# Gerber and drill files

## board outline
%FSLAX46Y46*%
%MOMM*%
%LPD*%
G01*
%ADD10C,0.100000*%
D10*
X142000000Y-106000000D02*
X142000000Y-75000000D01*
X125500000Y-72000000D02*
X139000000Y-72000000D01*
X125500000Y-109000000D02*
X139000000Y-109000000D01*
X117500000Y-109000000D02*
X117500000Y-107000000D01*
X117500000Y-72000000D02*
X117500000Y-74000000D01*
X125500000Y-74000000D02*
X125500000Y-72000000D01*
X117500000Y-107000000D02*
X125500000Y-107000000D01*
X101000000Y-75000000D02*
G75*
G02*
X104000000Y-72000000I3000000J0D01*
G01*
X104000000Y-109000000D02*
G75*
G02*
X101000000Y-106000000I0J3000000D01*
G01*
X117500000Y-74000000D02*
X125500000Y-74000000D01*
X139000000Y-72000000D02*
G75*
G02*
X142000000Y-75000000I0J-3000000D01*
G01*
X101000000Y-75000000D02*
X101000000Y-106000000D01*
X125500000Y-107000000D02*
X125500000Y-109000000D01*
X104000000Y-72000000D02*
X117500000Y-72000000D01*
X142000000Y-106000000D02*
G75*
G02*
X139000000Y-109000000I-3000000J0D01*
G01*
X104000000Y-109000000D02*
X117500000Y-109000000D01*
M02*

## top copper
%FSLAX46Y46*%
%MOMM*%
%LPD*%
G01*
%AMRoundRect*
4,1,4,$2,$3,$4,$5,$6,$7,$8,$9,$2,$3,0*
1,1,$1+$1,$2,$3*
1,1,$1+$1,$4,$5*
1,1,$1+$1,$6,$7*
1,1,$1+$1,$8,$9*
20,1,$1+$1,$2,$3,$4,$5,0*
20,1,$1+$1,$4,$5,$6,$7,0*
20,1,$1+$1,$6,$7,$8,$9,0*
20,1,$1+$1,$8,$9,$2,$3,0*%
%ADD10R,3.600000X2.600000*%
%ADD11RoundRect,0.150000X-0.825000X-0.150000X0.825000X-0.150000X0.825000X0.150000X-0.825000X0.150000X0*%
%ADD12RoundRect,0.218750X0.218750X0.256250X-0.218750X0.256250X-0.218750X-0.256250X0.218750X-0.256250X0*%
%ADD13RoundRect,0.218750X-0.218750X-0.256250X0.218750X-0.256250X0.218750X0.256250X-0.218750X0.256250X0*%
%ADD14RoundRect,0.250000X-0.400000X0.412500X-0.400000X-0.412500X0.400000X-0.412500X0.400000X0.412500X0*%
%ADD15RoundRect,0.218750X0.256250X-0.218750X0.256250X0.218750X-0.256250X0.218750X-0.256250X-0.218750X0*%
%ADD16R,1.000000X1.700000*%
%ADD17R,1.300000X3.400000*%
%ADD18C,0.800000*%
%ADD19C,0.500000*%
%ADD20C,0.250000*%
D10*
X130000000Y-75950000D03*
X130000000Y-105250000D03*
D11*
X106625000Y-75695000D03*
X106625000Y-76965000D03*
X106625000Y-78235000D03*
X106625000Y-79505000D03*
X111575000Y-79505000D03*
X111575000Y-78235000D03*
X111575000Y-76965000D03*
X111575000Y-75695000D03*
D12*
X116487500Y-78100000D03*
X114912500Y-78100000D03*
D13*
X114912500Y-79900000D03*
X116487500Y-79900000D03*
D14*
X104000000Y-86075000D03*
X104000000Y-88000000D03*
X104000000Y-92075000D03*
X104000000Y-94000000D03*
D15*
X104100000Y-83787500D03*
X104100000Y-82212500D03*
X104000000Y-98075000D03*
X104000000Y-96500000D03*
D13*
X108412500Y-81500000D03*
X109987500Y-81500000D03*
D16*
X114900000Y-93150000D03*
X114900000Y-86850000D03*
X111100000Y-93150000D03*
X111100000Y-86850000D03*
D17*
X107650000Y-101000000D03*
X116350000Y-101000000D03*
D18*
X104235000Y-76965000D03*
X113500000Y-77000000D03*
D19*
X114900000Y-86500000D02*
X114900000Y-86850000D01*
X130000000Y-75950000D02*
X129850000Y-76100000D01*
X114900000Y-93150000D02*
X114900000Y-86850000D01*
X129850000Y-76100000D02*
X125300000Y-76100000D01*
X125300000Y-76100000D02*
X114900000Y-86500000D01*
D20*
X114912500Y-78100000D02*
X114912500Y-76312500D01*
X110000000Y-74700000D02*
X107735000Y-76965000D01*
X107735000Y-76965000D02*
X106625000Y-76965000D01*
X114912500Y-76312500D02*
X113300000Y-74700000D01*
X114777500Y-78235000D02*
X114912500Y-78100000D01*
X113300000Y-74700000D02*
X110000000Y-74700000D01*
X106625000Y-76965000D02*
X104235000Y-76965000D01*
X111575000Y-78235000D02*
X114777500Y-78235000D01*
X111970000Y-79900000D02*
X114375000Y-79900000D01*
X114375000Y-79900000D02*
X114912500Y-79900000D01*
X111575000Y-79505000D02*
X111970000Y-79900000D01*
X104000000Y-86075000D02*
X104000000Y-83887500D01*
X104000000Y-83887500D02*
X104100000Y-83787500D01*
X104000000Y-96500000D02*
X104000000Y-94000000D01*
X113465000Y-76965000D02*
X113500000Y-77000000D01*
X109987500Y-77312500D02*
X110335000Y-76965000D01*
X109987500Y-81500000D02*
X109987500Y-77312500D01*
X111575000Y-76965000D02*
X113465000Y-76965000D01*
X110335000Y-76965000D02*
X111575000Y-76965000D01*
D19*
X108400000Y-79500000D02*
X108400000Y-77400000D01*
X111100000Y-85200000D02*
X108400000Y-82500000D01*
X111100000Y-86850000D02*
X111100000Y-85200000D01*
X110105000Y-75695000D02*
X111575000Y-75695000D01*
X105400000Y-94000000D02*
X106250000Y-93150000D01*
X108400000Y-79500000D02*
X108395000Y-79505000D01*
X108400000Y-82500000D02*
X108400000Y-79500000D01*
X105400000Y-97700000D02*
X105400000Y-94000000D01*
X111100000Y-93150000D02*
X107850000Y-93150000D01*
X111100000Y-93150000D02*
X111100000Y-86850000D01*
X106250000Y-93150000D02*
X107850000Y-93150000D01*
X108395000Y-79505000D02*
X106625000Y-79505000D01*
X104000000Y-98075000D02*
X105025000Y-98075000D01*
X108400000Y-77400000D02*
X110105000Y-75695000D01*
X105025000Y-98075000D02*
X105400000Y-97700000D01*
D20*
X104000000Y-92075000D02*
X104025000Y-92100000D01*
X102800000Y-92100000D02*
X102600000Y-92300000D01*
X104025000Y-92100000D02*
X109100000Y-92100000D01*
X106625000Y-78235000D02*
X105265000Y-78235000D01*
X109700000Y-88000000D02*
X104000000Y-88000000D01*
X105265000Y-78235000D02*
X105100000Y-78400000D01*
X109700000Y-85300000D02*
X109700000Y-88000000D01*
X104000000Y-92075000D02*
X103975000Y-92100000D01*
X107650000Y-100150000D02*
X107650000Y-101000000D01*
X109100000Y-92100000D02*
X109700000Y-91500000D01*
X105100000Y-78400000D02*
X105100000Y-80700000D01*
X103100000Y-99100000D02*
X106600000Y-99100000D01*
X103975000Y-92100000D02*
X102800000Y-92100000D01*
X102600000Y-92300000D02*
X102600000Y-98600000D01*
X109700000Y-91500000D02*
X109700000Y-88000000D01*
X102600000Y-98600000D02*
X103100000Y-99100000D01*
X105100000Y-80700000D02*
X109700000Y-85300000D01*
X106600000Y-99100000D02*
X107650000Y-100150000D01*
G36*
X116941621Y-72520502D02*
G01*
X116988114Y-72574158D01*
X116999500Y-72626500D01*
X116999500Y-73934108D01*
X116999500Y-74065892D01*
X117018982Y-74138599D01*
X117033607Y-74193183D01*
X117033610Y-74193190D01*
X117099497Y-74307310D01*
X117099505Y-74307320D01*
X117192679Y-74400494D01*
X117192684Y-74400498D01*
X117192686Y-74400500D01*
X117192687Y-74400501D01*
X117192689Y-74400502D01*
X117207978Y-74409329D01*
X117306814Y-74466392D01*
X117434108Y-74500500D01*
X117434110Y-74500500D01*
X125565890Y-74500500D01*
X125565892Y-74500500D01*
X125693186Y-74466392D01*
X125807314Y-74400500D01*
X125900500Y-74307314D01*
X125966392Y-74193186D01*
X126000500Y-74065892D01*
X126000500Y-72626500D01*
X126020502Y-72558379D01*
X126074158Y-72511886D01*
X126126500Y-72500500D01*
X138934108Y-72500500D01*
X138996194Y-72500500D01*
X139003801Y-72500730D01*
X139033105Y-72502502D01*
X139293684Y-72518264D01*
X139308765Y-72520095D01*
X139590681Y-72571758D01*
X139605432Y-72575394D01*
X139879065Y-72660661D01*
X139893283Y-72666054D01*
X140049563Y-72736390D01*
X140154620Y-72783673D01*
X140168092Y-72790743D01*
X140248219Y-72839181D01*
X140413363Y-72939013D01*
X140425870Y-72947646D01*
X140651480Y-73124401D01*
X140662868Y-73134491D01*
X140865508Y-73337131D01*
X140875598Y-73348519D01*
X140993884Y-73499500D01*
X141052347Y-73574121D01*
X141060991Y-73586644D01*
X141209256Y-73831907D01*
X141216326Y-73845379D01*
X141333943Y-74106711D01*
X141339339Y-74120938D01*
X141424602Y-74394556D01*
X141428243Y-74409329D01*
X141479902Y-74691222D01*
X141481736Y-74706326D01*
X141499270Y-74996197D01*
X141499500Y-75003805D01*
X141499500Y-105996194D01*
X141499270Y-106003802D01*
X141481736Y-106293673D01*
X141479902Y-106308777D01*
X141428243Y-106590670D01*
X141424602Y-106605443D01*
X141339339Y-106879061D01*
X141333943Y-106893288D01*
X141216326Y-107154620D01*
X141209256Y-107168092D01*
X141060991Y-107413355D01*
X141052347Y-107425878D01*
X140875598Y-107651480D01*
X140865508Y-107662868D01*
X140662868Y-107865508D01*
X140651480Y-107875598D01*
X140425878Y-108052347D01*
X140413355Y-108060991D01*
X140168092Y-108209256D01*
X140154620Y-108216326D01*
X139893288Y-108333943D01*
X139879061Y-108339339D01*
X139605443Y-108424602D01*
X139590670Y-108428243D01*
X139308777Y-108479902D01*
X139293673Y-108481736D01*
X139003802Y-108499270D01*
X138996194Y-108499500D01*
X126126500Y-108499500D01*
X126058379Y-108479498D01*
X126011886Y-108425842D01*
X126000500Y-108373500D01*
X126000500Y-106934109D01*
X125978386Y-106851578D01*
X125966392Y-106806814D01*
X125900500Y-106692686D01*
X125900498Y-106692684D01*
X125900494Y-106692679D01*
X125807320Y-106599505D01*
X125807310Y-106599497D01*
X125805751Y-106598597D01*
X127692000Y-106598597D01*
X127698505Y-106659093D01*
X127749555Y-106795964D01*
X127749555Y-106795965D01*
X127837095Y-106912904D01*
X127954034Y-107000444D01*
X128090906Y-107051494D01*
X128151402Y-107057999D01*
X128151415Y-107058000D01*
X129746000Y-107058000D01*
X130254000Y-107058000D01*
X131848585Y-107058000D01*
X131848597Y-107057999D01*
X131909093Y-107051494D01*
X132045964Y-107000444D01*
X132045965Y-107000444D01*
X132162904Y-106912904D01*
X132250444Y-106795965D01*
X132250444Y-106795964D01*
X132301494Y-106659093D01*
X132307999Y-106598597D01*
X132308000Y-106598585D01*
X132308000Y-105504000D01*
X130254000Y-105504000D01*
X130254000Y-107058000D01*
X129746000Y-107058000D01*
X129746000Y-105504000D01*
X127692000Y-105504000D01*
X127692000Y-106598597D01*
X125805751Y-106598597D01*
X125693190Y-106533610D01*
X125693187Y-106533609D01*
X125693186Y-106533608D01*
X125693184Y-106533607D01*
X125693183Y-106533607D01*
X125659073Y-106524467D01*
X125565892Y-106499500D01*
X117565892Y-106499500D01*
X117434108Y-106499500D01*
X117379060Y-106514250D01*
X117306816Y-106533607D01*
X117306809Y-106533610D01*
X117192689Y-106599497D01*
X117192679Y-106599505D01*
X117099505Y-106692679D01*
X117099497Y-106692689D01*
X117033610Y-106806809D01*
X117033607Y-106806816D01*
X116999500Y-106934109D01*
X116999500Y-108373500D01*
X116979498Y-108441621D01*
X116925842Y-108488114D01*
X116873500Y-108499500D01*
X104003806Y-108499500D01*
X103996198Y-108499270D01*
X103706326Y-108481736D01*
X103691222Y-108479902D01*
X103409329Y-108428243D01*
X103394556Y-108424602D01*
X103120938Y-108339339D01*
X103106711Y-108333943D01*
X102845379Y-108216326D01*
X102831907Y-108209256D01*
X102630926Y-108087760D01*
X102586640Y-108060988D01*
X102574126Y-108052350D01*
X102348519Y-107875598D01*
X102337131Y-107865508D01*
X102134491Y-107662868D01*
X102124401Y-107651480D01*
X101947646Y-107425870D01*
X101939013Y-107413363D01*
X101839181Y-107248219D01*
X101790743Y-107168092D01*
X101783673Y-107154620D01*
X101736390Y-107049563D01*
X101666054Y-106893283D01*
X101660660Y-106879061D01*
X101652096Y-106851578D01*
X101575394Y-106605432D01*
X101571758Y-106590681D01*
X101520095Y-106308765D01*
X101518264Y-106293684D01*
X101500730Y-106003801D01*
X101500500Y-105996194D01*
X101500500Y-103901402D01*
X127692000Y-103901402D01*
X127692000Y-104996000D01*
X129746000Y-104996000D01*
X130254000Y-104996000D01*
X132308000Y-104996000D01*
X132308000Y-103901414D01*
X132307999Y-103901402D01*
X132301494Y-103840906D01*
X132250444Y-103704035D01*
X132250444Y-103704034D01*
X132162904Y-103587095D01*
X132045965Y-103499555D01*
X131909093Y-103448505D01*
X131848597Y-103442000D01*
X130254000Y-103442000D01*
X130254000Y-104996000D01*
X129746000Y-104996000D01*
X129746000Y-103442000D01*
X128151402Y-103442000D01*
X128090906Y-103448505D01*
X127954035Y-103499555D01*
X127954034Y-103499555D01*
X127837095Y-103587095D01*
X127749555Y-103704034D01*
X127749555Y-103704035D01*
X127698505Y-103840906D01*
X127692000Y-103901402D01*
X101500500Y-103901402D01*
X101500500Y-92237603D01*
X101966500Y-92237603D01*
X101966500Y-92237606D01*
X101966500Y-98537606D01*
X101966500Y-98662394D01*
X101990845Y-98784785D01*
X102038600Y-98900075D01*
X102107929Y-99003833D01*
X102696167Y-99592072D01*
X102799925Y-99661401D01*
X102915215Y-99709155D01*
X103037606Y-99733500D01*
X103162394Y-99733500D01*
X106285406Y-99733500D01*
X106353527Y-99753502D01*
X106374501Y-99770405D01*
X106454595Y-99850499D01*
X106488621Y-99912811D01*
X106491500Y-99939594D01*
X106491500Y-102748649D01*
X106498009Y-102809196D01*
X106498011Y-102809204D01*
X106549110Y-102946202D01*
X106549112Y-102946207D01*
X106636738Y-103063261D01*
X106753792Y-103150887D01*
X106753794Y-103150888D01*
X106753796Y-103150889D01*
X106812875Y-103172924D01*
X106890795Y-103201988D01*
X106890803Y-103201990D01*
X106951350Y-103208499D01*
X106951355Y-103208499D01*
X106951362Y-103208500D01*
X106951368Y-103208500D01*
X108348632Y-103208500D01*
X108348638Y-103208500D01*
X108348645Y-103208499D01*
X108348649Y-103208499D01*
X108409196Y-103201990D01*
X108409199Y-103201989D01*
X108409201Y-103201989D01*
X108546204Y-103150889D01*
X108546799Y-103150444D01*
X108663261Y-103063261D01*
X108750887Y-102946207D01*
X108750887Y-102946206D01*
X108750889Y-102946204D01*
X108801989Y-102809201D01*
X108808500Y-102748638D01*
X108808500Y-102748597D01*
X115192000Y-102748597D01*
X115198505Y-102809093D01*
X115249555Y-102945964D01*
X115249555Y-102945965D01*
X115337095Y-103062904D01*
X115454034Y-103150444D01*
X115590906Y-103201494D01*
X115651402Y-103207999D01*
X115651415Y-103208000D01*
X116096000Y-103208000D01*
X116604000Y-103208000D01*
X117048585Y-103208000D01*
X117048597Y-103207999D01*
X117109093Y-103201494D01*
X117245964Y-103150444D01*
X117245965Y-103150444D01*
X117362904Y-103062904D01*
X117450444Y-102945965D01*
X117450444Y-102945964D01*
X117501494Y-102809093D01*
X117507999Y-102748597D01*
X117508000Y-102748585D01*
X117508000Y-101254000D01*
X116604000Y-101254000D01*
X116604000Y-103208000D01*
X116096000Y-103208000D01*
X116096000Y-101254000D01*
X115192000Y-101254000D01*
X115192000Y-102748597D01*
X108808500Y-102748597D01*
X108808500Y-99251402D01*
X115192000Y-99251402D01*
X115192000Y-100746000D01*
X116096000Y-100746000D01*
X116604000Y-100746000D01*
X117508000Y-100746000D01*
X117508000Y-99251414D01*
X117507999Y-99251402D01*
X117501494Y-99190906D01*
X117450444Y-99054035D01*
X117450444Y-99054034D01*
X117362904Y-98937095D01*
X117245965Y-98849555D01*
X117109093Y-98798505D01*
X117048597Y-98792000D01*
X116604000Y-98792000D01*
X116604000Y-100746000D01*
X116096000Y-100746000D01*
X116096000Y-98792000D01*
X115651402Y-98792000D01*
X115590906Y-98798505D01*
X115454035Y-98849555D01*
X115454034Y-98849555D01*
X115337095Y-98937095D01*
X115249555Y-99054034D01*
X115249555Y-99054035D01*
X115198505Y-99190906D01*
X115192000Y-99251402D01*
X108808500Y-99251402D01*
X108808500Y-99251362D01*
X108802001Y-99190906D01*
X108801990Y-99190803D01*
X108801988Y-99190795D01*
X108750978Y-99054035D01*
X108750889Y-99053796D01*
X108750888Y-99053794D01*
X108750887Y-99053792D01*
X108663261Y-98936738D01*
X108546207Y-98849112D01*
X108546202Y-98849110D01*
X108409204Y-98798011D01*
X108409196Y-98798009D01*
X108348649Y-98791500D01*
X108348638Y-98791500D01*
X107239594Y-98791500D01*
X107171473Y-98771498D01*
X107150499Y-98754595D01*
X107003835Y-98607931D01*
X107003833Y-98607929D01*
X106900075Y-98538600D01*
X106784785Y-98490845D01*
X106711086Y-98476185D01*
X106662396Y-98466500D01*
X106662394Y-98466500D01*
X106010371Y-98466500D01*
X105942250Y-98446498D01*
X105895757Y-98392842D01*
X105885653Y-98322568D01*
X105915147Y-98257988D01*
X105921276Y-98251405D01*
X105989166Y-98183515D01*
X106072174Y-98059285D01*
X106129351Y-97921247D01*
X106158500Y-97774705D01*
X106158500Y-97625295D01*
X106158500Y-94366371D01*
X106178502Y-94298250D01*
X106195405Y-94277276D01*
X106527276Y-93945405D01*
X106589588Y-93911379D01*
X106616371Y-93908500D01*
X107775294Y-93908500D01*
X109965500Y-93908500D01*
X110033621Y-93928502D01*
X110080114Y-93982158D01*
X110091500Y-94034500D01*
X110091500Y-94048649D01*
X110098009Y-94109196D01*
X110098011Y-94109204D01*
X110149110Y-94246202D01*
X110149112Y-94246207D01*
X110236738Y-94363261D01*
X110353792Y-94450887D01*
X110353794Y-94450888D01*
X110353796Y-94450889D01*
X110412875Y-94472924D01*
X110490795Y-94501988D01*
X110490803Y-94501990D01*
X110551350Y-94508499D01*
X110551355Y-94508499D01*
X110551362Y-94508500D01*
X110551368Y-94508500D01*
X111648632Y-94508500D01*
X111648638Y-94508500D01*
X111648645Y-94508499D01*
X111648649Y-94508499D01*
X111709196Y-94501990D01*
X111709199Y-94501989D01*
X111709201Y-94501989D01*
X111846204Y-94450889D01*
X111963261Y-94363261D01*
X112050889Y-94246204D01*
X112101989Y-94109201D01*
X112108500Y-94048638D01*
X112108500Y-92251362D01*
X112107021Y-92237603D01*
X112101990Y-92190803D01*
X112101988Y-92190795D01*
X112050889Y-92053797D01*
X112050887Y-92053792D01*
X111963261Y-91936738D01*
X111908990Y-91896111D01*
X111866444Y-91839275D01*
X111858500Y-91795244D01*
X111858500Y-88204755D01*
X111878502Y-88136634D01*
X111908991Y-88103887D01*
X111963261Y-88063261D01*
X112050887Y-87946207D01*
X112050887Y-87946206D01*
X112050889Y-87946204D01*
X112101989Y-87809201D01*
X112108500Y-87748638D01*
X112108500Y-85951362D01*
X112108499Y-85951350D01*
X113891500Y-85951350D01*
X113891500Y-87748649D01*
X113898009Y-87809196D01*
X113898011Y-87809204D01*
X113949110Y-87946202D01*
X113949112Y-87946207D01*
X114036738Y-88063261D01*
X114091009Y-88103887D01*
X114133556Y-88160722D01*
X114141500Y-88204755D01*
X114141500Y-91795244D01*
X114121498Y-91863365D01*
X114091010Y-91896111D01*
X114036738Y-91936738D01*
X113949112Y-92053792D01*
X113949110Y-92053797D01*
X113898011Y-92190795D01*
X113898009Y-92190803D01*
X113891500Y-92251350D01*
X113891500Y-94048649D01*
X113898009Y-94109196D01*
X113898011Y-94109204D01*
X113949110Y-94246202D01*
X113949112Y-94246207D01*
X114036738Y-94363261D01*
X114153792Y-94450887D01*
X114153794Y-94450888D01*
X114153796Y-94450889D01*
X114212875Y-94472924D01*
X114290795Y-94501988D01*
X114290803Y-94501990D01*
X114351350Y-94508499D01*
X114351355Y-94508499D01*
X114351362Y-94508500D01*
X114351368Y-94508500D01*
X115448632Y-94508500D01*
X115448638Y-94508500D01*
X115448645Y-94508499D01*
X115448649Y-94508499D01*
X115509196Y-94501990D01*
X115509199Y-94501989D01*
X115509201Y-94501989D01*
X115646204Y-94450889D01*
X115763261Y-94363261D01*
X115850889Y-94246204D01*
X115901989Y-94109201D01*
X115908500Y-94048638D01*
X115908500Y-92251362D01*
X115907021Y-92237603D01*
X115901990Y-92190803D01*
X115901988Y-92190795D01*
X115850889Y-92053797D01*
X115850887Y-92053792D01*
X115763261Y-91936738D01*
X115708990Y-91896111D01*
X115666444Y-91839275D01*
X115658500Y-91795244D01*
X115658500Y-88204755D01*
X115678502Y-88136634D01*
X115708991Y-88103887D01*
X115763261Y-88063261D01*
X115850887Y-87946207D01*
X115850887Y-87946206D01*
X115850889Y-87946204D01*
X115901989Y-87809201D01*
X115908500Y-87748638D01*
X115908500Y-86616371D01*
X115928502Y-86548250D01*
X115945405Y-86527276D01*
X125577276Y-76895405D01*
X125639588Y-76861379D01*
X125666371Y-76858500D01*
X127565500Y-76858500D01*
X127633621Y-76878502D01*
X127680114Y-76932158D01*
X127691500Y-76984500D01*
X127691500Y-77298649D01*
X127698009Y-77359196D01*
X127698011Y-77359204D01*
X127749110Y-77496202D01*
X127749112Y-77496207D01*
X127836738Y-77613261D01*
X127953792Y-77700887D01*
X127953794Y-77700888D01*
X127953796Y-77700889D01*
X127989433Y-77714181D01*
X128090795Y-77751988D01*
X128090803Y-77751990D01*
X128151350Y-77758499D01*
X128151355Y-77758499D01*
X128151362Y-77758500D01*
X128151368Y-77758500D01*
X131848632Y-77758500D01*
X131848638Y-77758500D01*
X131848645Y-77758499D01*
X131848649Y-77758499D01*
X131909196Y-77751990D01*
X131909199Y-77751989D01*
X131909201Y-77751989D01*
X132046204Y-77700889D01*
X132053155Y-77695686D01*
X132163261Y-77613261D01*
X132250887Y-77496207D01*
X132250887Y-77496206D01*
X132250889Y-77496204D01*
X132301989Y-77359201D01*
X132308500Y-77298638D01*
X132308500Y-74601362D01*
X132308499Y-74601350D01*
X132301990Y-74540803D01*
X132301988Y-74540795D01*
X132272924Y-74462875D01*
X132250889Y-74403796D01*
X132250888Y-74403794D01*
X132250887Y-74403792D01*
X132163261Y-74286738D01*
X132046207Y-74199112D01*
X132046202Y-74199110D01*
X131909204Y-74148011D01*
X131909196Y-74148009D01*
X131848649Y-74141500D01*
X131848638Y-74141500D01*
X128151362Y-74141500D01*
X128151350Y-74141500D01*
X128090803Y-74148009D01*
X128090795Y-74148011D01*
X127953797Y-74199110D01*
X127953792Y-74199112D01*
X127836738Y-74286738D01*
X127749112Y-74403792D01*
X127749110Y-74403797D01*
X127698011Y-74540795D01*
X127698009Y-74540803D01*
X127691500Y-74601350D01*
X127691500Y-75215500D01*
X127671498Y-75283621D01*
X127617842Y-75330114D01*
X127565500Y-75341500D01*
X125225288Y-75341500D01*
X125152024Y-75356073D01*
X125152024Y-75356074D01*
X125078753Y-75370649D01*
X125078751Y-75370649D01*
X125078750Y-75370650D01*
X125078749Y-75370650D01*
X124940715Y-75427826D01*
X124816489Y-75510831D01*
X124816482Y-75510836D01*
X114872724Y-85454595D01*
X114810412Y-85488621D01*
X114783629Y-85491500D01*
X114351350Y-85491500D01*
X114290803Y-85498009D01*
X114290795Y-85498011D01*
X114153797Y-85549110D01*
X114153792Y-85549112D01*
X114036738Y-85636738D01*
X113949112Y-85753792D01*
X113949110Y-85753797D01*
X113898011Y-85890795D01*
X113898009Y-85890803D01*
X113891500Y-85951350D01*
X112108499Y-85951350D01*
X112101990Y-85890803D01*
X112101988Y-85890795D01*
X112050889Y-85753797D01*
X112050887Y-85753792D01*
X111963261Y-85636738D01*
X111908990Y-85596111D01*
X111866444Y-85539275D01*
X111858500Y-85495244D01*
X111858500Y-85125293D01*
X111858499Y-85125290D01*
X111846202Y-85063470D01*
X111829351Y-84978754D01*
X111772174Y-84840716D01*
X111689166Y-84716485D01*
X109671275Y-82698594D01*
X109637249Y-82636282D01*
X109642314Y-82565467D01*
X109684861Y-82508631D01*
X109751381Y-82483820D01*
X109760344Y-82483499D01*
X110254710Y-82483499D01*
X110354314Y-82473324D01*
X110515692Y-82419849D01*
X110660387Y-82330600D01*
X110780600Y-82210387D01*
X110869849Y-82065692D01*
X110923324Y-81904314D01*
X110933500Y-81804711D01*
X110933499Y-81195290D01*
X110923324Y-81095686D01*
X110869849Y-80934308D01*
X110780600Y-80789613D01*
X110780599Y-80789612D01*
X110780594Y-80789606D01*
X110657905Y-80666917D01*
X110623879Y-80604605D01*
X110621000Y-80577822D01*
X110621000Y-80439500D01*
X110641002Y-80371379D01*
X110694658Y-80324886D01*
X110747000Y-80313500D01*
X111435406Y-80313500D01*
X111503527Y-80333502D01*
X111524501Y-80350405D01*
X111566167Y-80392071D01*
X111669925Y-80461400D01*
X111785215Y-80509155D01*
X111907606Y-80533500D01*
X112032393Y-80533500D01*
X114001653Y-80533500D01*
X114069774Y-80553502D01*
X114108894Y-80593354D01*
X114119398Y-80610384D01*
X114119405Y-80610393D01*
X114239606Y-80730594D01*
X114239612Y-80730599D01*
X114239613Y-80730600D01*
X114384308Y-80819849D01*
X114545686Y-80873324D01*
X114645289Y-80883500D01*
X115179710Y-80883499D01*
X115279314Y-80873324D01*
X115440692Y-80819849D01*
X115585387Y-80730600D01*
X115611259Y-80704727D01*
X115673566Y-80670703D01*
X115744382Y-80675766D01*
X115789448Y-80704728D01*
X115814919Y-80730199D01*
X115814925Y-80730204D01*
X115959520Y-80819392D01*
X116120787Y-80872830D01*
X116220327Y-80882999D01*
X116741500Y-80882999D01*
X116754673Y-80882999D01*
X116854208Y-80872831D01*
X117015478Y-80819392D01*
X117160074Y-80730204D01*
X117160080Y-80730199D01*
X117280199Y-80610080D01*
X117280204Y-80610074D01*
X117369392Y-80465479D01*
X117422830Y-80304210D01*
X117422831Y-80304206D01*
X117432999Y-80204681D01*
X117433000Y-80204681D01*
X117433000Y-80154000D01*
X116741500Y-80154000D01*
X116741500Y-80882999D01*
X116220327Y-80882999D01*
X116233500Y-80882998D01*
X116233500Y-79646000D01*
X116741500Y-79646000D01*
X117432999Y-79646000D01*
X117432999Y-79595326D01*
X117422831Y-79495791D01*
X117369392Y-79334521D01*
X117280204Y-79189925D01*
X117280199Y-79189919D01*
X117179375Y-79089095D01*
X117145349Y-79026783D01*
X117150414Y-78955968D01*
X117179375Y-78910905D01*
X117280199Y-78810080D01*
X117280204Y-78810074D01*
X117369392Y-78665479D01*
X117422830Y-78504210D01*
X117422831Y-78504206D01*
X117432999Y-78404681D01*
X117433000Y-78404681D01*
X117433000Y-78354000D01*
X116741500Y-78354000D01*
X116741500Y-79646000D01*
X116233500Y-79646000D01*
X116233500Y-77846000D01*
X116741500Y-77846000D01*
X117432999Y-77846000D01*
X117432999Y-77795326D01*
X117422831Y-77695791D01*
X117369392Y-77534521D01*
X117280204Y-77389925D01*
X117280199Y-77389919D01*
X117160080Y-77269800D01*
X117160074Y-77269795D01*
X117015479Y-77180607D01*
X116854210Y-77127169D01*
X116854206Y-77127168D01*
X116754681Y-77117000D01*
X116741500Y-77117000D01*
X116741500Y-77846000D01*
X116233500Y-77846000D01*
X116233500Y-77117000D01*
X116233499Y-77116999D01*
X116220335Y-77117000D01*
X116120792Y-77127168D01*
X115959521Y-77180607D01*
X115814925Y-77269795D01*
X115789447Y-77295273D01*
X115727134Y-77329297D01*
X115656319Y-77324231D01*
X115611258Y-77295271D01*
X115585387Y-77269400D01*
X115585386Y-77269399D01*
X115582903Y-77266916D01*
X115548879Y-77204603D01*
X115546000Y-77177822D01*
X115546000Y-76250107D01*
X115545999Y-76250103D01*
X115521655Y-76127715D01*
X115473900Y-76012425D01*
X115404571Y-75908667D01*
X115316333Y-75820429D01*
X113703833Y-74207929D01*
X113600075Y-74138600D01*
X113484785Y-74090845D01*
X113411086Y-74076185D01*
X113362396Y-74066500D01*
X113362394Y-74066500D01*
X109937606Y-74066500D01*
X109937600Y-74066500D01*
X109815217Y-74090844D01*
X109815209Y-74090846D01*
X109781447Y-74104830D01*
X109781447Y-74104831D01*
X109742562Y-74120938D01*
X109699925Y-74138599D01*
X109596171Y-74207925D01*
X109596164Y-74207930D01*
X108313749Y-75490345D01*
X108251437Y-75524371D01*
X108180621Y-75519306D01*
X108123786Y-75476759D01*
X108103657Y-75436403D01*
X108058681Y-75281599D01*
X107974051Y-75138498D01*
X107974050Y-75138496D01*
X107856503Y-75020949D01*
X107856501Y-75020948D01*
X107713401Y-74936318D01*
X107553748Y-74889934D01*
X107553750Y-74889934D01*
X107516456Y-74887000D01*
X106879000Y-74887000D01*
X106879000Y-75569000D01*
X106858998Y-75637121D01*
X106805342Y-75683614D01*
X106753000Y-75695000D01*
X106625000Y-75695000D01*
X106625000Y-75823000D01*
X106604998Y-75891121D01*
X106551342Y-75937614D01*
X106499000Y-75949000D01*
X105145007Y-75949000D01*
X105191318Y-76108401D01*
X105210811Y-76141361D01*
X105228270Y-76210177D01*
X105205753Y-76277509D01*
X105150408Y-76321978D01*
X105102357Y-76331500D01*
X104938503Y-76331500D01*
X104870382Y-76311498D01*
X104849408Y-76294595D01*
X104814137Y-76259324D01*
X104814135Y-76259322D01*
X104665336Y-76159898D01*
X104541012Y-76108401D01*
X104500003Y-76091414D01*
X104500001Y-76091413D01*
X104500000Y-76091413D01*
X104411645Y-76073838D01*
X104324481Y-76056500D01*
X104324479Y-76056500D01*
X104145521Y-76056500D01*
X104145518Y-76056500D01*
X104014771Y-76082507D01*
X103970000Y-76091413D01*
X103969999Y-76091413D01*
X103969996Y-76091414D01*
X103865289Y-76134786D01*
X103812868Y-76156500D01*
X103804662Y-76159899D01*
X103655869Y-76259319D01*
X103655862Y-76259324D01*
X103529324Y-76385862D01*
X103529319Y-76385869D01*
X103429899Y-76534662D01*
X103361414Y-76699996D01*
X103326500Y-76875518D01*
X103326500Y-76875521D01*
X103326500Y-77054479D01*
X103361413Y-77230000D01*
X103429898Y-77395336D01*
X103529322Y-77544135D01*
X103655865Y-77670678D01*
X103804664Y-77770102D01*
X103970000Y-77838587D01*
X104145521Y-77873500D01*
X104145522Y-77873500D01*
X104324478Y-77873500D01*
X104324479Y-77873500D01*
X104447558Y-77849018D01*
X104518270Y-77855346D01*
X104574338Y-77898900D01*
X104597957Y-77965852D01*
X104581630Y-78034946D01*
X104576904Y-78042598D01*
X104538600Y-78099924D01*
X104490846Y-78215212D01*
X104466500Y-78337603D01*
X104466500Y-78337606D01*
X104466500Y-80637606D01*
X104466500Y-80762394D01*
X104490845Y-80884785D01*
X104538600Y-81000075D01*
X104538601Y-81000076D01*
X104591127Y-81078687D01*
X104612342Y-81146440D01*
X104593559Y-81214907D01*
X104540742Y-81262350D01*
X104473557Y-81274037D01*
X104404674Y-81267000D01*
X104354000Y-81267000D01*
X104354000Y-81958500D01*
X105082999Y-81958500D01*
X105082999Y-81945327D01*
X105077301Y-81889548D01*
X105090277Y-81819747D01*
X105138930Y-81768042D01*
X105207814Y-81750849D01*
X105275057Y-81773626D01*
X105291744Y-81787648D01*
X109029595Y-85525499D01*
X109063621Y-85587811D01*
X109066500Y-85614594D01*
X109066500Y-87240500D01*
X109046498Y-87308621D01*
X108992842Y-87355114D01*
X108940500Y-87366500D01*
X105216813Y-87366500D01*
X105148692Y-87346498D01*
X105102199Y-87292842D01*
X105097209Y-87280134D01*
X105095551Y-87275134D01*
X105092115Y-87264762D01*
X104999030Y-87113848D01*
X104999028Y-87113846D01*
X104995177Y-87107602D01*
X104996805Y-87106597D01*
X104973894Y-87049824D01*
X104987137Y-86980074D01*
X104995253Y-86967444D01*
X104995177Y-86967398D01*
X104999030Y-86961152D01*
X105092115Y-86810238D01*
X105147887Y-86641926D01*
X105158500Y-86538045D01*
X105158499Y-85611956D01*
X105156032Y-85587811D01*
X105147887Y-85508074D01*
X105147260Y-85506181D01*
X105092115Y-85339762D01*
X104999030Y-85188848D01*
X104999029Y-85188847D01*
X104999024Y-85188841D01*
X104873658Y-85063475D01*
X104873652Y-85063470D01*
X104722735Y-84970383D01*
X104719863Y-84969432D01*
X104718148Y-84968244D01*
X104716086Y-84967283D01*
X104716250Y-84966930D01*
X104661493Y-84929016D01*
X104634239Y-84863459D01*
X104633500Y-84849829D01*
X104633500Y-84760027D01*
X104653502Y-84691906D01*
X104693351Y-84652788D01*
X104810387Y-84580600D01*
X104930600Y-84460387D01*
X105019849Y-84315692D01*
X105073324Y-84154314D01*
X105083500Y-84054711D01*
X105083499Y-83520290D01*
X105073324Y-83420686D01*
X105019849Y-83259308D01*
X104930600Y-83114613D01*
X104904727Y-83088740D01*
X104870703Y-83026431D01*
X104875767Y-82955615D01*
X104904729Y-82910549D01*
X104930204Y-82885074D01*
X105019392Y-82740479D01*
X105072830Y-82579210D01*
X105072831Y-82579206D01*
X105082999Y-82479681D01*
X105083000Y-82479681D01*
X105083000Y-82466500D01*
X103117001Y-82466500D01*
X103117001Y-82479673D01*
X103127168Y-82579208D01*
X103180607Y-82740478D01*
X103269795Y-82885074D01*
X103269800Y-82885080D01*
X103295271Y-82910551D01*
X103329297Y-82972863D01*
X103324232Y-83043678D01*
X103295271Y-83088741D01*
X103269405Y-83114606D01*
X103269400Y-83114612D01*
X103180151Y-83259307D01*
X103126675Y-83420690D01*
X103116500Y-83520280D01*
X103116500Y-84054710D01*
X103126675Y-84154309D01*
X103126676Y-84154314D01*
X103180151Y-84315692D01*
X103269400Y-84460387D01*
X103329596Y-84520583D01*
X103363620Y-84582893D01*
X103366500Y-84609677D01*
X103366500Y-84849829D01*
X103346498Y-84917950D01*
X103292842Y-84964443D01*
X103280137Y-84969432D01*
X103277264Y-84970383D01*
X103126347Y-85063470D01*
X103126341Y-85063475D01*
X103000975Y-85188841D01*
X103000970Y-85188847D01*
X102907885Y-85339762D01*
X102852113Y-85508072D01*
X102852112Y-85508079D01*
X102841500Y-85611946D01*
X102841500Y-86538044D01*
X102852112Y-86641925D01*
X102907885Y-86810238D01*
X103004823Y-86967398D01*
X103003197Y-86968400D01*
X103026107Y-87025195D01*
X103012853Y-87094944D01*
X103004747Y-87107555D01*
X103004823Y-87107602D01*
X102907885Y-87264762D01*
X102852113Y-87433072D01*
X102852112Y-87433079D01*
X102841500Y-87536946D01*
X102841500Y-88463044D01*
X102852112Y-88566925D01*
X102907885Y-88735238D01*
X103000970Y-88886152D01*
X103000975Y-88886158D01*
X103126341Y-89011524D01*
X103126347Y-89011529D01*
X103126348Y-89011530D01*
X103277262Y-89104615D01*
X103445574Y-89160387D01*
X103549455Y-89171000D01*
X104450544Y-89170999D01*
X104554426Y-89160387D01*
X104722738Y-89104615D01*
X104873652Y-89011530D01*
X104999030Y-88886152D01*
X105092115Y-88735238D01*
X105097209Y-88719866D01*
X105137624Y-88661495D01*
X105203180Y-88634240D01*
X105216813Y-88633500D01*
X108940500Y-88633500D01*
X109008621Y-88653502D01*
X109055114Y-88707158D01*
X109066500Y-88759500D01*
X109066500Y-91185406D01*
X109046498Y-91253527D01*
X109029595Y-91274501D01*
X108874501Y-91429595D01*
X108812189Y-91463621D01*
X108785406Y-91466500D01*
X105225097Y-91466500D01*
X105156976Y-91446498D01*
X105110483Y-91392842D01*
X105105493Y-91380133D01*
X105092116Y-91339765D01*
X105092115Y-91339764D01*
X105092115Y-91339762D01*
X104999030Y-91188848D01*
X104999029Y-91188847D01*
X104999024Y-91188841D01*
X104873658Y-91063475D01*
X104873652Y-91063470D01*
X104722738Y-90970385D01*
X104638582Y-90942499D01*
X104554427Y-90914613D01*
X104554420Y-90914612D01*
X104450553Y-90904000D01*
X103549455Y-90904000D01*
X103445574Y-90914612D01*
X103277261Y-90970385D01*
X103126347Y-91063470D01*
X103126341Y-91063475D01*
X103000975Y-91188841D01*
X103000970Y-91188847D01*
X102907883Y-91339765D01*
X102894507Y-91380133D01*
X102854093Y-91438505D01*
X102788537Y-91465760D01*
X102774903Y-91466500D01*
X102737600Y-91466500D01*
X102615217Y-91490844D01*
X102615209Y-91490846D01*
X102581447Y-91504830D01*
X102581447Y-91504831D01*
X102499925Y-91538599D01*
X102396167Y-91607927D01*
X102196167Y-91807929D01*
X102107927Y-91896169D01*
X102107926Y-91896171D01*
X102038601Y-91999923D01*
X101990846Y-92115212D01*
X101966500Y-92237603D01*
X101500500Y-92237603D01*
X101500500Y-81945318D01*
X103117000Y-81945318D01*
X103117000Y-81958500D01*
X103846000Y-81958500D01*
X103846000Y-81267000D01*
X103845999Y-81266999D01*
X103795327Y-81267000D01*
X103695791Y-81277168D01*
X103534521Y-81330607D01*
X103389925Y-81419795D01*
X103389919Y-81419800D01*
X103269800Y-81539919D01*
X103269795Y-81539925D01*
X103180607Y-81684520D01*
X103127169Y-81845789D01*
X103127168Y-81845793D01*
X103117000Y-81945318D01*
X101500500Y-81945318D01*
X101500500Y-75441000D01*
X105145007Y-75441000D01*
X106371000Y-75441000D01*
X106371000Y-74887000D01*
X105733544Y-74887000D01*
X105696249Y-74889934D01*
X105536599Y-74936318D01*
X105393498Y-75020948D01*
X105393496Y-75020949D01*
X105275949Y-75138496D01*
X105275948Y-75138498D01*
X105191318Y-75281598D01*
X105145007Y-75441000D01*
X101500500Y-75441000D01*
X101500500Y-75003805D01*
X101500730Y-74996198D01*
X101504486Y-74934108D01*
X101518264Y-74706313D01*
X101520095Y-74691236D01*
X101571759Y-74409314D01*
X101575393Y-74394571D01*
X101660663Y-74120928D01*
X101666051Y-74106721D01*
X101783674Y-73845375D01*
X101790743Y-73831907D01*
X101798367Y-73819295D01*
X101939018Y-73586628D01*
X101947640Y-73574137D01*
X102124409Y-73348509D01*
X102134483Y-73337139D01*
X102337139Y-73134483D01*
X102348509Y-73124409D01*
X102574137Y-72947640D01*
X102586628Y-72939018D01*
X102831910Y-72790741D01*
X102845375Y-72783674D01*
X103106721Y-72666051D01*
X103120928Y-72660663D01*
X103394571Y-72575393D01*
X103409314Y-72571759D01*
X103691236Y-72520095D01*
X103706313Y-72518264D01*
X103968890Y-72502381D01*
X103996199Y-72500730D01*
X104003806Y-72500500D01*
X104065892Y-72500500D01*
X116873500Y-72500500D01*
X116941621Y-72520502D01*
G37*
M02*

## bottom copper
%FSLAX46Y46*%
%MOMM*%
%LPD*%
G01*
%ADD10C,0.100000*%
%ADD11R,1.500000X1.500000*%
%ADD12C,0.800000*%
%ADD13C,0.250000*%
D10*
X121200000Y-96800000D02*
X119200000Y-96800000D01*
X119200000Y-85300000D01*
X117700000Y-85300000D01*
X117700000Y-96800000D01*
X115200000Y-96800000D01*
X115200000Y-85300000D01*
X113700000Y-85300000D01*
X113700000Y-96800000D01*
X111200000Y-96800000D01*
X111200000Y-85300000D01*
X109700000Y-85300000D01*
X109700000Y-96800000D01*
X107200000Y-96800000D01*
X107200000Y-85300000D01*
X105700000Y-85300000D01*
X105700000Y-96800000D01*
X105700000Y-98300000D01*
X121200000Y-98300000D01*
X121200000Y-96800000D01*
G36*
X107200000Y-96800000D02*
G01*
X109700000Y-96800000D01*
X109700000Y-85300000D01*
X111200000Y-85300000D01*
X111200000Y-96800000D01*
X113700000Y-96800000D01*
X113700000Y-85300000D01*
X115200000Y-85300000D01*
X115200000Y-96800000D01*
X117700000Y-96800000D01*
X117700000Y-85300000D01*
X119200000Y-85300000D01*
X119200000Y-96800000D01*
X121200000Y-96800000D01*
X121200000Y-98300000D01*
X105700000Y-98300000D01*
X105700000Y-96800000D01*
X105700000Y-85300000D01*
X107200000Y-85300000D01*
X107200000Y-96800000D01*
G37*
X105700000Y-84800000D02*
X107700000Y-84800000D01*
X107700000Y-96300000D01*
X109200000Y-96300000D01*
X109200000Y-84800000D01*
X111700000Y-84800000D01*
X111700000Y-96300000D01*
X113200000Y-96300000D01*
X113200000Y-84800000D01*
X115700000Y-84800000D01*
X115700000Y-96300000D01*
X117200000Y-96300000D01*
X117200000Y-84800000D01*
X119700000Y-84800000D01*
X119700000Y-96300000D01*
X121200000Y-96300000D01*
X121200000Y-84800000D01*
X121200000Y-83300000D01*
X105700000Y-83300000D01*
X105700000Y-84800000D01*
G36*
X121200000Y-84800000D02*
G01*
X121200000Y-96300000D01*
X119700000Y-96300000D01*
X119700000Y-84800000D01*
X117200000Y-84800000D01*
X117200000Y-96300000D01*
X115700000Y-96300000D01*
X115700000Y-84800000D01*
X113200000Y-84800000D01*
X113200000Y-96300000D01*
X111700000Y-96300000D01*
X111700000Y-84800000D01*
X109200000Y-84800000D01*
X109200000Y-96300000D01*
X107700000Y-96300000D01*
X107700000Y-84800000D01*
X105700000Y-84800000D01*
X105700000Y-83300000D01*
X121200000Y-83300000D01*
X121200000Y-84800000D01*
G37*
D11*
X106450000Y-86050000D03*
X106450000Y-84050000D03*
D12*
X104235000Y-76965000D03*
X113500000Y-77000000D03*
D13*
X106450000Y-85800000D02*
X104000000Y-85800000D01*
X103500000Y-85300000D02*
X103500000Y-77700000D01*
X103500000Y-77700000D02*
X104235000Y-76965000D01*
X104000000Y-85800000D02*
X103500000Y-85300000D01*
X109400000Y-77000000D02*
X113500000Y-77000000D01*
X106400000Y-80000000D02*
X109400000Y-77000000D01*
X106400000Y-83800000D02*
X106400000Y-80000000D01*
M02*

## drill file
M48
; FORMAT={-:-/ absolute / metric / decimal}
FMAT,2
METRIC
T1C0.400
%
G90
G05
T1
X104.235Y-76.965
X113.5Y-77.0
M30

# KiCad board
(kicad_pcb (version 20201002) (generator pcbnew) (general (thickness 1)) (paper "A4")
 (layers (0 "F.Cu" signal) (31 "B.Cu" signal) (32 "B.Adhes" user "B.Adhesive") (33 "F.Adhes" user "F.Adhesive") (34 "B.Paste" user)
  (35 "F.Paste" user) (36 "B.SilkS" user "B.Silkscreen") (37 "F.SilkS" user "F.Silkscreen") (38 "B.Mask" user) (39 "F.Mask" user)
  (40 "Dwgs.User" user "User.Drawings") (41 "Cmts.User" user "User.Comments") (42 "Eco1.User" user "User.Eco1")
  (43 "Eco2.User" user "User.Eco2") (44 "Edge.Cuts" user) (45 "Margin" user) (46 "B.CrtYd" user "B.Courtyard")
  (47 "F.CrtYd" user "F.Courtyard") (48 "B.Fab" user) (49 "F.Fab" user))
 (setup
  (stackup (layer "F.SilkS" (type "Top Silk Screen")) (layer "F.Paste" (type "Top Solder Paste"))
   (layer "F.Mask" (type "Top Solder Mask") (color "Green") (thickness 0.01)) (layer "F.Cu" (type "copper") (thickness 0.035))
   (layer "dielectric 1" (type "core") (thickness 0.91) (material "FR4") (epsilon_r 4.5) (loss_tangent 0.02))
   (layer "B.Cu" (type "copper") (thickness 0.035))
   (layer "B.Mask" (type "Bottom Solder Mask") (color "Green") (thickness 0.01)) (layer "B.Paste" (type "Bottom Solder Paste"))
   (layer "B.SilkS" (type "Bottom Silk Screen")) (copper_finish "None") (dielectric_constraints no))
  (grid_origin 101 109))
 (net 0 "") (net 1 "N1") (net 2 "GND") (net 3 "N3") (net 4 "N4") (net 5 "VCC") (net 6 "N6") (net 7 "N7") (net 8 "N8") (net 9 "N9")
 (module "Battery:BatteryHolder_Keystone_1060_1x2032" (layer "F.Cu") (at 130 90.6 -90)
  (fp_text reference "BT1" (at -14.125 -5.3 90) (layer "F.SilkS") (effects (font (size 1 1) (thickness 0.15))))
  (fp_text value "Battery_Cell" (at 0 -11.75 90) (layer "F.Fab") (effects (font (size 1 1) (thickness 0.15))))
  (pad "1" smd rect (at -14.65 0 90) (size 2.6 3.6) (layers "F.Cu" "F.Paste" "F.Mask") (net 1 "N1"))
  (pad "2" smd rect (at 14.65 0 90) (size 2.6 3.6) (layers "F.Cu" "F.Paste" "F.Mask") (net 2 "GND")))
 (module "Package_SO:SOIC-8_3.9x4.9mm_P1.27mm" (layer "F.Cu") (at 109.1 77.6)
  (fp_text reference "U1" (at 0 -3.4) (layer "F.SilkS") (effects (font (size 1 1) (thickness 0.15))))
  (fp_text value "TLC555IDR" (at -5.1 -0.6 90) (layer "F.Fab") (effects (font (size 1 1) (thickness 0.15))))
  (pad "1" smd roundrect (at -2.475 -1.905) (size 1.95 0.6) (layers "F.Cu" "F.Paste" "F.Mask") (roundrect_rratio 0.25) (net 2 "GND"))
  (pad "2" smd roundrect (at -2.475 -0.635) (size 1.95 0.6) (layers "F.Cu" "F.Paste" "F.Mask") (roundrect_rratio 0.25) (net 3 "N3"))
  (pad "3" smd roundrect (at -2.475 0.635) (size 1.95 0.6) (layers "F.Cu" "F.Paste" "F.Mask") (roundrect_rratio 0.25) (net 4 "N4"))
  (pad "4" smd roundrect (at -2.475 1.905) (size 1.95 0.6) (layers "F.Cu" "F.Paste" "F.Mask") (roundrect_rratio 0.25) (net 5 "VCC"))
  (pad "5" smd roundrect (at 2.475 1.905) (size 1.95 0.6) (layers "F.Cu" "F.Paste" "F.Mask") (roundrect_rratio 0.25) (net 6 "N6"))
  (pad "6" smd roundrect (at 2.475 0.635) (size 1.95 0.6) (layers "F.Cu" "F.Paste" "F.Mask") (roundrect_rratio 0.25) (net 3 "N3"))
  (pad "7" smd roundrect (at 2.475 -0.635) (size 1.95 0.6) (layers "F.Cu" "F.Paste" "F.Mask") (roundrect_rratio 0.25) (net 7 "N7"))
  (pad "8" smd roundrect (at 2.475 -1.905) (size 1.95 0.6) (layers "F.Cu" "F.Paste" "F.Mask") (roundrect_rratio 0.25) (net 5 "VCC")))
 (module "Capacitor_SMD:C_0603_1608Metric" (layer "F.Cu") (at 115.7 78.1 180)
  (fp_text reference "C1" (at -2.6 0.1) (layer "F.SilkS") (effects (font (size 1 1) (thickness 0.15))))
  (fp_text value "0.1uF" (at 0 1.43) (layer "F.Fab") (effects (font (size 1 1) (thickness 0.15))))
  (pad "1" smd roundrect (at -0.7875 0 180) (size 0.875 0.95) (layers "F.Cu" "F.Paste" "F.Mask") (roundrect_rratio 0.25) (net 2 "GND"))
  (pad "2" smd roundrect (at 0.7875 0 180) (size 0.875 0.95) (layers "F.Cu" "F.Paste" "F.Mask") (roundrect_rratio 0.25) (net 3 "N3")))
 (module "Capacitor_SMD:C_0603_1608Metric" (layer "F.Cu") (at 115.7 79.9)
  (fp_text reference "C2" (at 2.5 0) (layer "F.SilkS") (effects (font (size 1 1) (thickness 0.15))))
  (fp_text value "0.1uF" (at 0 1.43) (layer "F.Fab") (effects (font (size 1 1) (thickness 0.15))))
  (pad "1" smd roundrect (at -0.7875 0) (size 0.875 0.95) (layers "F.Cu" "F.Paste" "F.Mask") (roundrect_rratio 0.25) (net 6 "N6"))
  (pad "2" smd roundrect (at 0.7875 0) (size 0.875 0.95) (layers "F.Cu" "F.Paste" "F.Mask") (roundrect_rratio 0.25) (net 2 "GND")))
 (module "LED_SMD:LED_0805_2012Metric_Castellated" (layer "F.Cu") (at 104 87.0375 -90)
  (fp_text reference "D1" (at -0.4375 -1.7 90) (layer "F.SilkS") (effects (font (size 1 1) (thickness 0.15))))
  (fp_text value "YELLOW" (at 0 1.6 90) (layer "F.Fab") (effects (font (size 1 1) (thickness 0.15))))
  (pad "1" smd roundrect (at -0.9625 0 270) (size 1.325 1.3) (layers "F.Cu" "F.Paste" "F.Mask") (roundrect_rratio 0.192308) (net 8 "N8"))
  (pad "2" smd roundrect (at 0.9625 0 270) (size 1.325 1.3) (layers "F.Cu" "F.Paste" "F.Mask") (roundrect_rratio 0.192308) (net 4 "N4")))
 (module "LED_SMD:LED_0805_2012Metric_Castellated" (layer "F.Cu") (at 104 93.0375 -90)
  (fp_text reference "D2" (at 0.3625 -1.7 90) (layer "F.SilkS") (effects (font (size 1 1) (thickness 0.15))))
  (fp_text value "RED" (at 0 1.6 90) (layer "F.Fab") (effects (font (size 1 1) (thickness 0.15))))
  (pad "1" smd roundrect (at -0.9625 0 270) (size 1.325 1.3) (layers "F.Cu" "F.Paste" "F.Mask") (roundrect_rratio 0.192308) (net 4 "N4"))
  (pad "2" smd roundrect (at 0.9625 0 270) (size 1.325 1.3) (layers "F.Cu" "F.Paste" "F.Mask") (roundrect_rratio 0.192308) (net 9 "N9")))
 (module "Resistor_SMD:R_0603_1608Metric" (layer "F.Cu") (at 104.1 83 90)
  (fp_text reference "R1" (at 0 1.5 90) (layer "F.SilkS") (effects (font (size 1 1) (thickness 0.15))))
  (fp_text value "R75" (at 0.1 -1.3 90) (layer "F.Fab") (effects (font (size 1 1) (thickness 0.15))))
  (pad "1" smd roundrect (at -0.7875 0 90) (size 0.875 0.95) (layers "F.Cu" "F.Paste" "F.Mask") (roundrect_rratio 0.25) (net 8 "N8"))
  (pad "2" smd roundrect (at 0.7875 0 90) (size 0.875 0.95) (layers "F.Cu" "F.Paste" "F.Mask") (roundrect_rratio 0.25) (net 2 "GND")))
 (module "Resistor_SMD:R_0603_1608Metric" (layer "F.Cu") (at 104 97.2875 90)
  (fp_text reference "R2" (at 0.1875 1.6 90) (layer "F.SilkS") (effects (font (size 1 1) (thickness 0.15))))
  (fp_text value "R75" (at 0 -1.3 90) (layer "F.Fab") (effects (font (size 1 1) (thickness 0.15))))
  (pad "1" smd roundrect (at -0.7875 0 90) (size 0.875 0.95) (layers "F.Cu" "F.Paste" "F.Mask") (roundrect_rratio 0.25) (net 5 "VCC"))
  (pad "2" smd roundrect (at 0.7875 0 90) (size 0.875 0.95) (layers "F.Cu" "F.Paste" "F.Mask") (roundrect_rratio 0.25) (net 9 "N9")))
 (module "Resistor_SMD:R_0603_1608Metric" (layer "F.Cu") (at 109.2 81.5)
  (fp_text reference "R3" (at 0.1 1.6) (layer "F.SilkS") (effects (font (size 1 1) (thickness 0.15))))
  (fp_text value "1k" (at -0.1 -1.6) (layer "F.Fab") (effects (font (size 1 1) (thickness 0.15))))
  (pad "1" smd roundrect (at -0.7875 0) (size 0.875 0.95) (layers "F.Cu" "F.Paste" "F.Mask") (roundrect_rratio 0.25) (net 5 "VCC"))
  (pad "2" smd roundrect (at 0.7875 0) (size 0.875 0.95) (layers "F.Cu" "F.Paste" "F.Mask") (roundrect_rratio 0.25) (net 7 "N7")))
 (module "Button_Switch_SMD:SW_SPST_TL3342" (layer "F.Cu") (at 113 90 -90)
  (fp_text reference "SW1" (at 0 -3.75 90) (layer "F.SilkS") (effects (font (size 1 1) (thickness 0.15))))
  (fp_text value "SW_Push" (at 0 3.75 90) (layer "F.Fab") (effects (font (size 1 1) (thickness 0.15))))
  (pad "1" smd rect (at 3.15 -1.9 270) (size 1.7 1) (layers "F.Cu" "F.Paste" "F.Mask") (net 1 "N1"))
  (pad "1" smd rect (at -3.15 -1.9 270) (size 1.7 1) (layers "F.Cu" "F.Paste" "F.Mask") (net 1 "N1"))
  (pad "2" smd rect (at 3.15 1.9 270) (size 1.7 1) (layers "F.Cu" "F.Paste" "F.Mask") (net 5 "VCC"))
  (pad "2" smd rect (at -3.15 1.9 270) (size 1.7 1) (layers "F.Cu" "F.Paste" "F.Mask") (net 5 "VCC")))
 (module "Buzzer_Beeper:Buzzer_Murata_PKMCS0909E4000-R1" (layer "F.Cu") (at 112 101)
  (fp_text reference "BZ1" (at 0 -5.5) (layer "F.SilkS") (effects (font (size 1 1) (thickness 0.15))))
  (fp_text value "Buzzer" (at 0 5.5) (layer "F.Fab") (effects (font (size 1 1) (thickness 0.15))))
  (pad "1" smd rect (at -4.35 0) (size 1.3 3.4) (layers "F.Cu" "F.Paste" "F.Mask") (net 4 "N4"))
  (pad "2" smd rect (at 4.35 0) (size 1.3 3.4) (layers "F.Cu" "F.Paste" "F.Mask") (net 2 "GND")))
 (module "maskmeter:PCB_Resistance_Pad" (layer "B.Cu") (at 113.7 89.8)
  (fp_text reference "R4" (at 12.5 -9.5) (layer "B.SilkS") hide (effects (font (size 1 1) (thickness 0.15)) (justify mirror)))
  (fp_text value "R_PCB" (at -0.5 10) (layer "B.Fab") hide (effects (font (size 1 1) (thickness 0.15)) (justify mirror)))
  (fp_poly
   (pts (xy 7.5 7) (xy 5.5 7) (xy 5.5 -4.5) (xy 4 -4.5) (xy 4 7) (xy 1.5 7) (xy 1.5 -4.5) (xy 0 -4.5) (xy 0 7) (xy -2.5 7) (xy -2.5 -4.5)
    (xy -4 -4.5) (xy -4 7) (xy -6.5 7) (xy -6.5 -4.5) (xy -8 -4.5) (xy -8 7) (xy -8 8.5) (xy 7.5 8.5))
   (layer "B.Cu") (width 0.1))
  (fp_poly
   (pts (xy -8 -5) (xy -6 -5) (xy -6 6.5) (xy -4.5 6.5) (xy -4.5 -5) (xy -2 -5) (xy -2 6.5) (xy -0.5 6.5) (xy -0.5 -5) (xy 2 -5) (xy 2 6.5)
    (xy 3.5 6.5) (xy 3.5 -5) (xy 6 -5) (xy 6 6.5) (xy 7.5 6.5) (xy 7.5 -5) (xy 7.5 -6.5) (xy -8 -6.5))
   (layer "B.Cu") (width 0.1))
  (pad "1" smd rect (at -7.25 -3.75) (size 1.5 1.5) (layers "B.Cu" "B.Mask") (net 3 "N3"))
  (pad "2" smd rect (at -7.25 -5.75) (size 1.5 1.5) (layers "B.Cu" "B.Mask") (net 7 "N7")))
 (gr_line (start 142 106) (end 142 75) (layer "Edge.Cuts") (width 0.1))
 (gr_line (start 125.5 72) (end 139 72) (layer "Edge.Cuts") (width 0.1))
 (gr_line (start 125.5 109) (end 139 109) (layer "Edge.Cuts") (width 0.1))
 (gr_line (start 117.5 109) (end 117.5 107) (layer "Edge.Cuts") (width 0.1))
 (gr_line (start 117.5 72) (end 117.5 74) (layer "Edge.Cuts") (width 0.1))
 (gr_line (start 125.5 74) (end 125.5 72) (layer "Edge.Cuts") (width 0.1))
 (gr_line (start 117.5 107) (end 125.5 107) (layer "Edge.Cuts") (width 0.1))
 (gr_arc (start 104 75) (end 104 72) (angle -90) (layer "Edge.Cuts") (width 0.1))
 (gr_arc (start 104 106) (end 101 106) (angle -90) (layer "Edge.Cuts") (width 0.1))
 (gr_line (start 117.5 74) (end 125.5 74) (layer "Edge.Cuts") (width 0.1))
 (gr_arc (start 139 75) (end 142 75) (angle -90) (layer "Edge.Cuts") (width 0.1))
 (gr_line (start 101 75) (end 101 106) (layer "Edge.Cuts") (width 0.1))
 (gr_line (start 125.5 107) (end 125.5 109) (layer "Edge.Cuts") (width 0.1))
 (gr_line (start 104 72) (end 117.5 72) (layer "Edge.Cuts") (width 0.1))
 (gr_arc (start 139 106) (end 139 109) (angle -90) (layer "Edge.Cuts") (width 0.1))
 (gr_line (start 104 109) (end 117.5 109) (layer "Edge.Cuts") (width 0.1))
 (segment (start 114.9 86.5) (end 114.9 86.85) (width 0.5) (layer "F.Cu") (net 1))
 (segment (start 130 75.95) (end 129.85 76.1) (width 0.5) (layer "F.Cu") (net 1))
 (segment (start 114.9 93.15) (end 114.9 86.85) (width 0.5) (layer "F.Cu") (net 1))
 (segment (start 129.85 76.1) (end 125.3 76.1) (width 0.5) (layer "F.Cu") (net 1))
 (segment (start 125.3 76.1) (end 114.9 86.5) (width 0.5) (layer "F.Cu") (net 1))
 (segment (start 114.9125 78.1) (end 114.9125 76.3125) (width 0.25) (layer "F.Cu") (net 3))
 (segment (start 110 74.7) (end 107.735 76.965) (width 0.25) (layer "F.Cu") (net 3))
 (segment (start 107.735 76.965) (end 106.625 76.965) (width 0.25) (layer "F.Cu") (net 3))
 (segment (start 114.9125 76.3125) (end 113.3 74.7) (width 0.25) (layer "F.Cu") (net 3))
 (segment (start 114.7775 78.235) (end 114.9125 78.1) (width 0.25) (layer "F.Cu") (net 3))
 (segment (start 113.3 74.7) (end 110 74.7) (width 0.25) (layer "F.Cu") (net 3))
 (segment (start 106.625 76.965) (end 104.235 76.965) (width 0.25) (layer "F.Cu") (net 3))
 (segment (start 111.575 78.235) (end 114.7775 78.235) (width 0.25) (layer "F.Cu") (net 3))
 (via (at 104.235 76.965) (size 0.8) (drill 0.4) (layers "F.Cu" "B.Cu") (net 3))
 (segment (start 106.45 85.8) (end 104 85.8) (width 0.25) (layer "B.Cu") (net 3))
 (segment (start 103.5 85.3) (end 103.5 77.7) (width 0.25) (layer "B.Cu") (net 3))
 (segment (start 103.5 77.7) (end 104.235 76.965) (width 0.25) (layer "B.Cu") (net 3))
 (segment (start 104 85.8) (end 103.5 85.3) (width 0.25) (layer "B.Cu") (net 3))
 (segment (start 111.97 79.9) (end 114.375 79.9) (width 0.25) (layer "F.Cu") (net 6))
 (segment (start 114.375 79.9) (end 114.9125 79.9) (width 0.25) (layer "F.Cu") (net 6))
 (segment (start 111.575 79.505) (end 111.97 79.9) (width 0.25) (layer "F.Cu") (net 6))
 (segment (start 104 86.075) (end 104 83.8875) (width 0.25) (layer "F.Cu") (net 8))
 (segment (start 104 83.8875) (end 104.1 83.7875) (width 0.25) (layer "F.Cu") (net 8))
 (segment (start 104 96.5) (end 104 94) (width 0.25) (layer "F.Cu") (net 9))
 (segment (start 113.465 76.965) (end 113.5 77) (width 0.25) (layer "F.Cu") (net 7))
 (segment (start 109.9875 77.3125) (end 110.335 76.965) (width 0.25) (layer "F.Cu") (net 7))
 (segment (start 109.9875 81.5) (end 109.9875 77.3125) (width 0.25) (layer "F.Cu") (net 7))
 (segment (start 111.575 76.965) (end 113.465 76.965) (width 0.25) (layer "F.Cu") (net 7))
 (segment (start 110.335 76.965) (end 111.575 76.965) (width 0.25) (layer "F.Cu") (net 7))
 (via (at 113.5 77) (size 0.8) (drill 0.4) (layers "F.Cu" "B.Cu") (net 7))
 (segment (start 109.4 77) (end 113.5 77) (width 0.25) (layer "B.Cu") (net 7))
 (segment (start 106.4 80) (end 109.4 77) (width 0.25) (layer "B.Cu") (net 7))
 (segment (start 106.4 83.8) (end 106.4 80) (width 0.25) (layer "B.Cu") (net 7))
 (segment (start 108.4 79.5) (end 108.4 77.4) (width 0.5) (layer "F.Cu") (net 5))
 (segment (start 111.1 85.2) (end 108.4 82.5) (width 0.5) (layer "F.Cu") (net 5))
 (segment (start 111.1 86.85) (end 111.1 85.2) (width 0.5) (layer "F.Cu") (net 5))
 (segment (start 110.105 75.695) (end 111.575 75.695) (width 0.5) (layer "F.Cu") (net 5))
 (segment (start 105.4 94) (end 106.25 93.15) (width 0.5) (layer "F.Cu") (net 5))
 (segment (start 108.4 79.5) (end 108.395 79.505) (width 0.5) (layer "F.Cu") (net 5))
 (segment (start 108.4 82.5) (end 108.4 79.5) (width 0.5) (layer "F.Cu") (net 5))
 (segment (start 105.4 97.7) (end 105.4 94) (width 0.5) (layer "F.Cu") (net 5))
 (segment (start 111.1 93.15) (end 107.85 93.15) (width 0.5) (layer "F.Cu") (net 5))
 (segment (start 111.1 93.15) (end 111.1 86.85) (width 0.5) (layer "F.Cu") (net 5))
 (segment (start 106.25 93.15) (end 107.85 93.15) (width 0.5) (layer "F.Cu") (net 5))
 (segment (start 108.395 79.505) (end 106.625 79.505) (width 0.5) (layer "F.Cu") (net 5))
 (segment (start 104 98.075) (end 105.025 98.075) (width 0.5) (layer "F.Cu") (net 5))
 (segment (start 108.4 77.4) (end 110.105 75.695) (width 0.5) (layer "F.Cu") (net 5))
 (segment (start 105.025 98.075) (end 105.4 97.7) (width 0.5) (layer "F.Cu") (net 5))
 (segment (start 104 92.075) (end 104.025 92.1) (width 0.25) (layer "F.Cu") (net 4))
 (segment (start 102.8 92.1) (end 102.6 92.3) (width 0.25) (layer "F.Cu") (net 4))
 (segment (start 104.025 92.1) (end 109.1 92.1) (width 0.25) (layer "F.Cu") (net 4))
 (segment (start 106.625 78.235) (end 105.265 78.235) (width 0.25) (layer "F.Cu") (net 4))
 (segment (start 109.7 88) (end 104 88) (width 0.25) (layer "F.Cu") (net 4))
 (segment (start 105.265 78.235) (end 105.1 78.4) (width 0.25) (layer "F.Cu") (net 4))
 (segment (start 109.7 85.3) (end 109.7 88) (width 0.25) (layer "F.Cu") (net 4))
 (segment (start 104 92.075) (end 103.975 92.1) (width 0.25) (layer "F.Cu") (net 4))
 (segment (start 107.65 100.15) (end 107.65 101) (width 0.25) (layer "F.Cu") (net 4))
 (segment (start 109.1 92.1) (end 109.7 91.5) (width 0.25) (layer "F.Cu") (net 4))
 (segment (start 105.1 78.4) (end 105.1 80.7) (width 0.25) (layer "F.Cu") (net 4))
 (segment (start 103.1 99.1) (end 106.6 99.1) (width 0.25) (layer "F.Cu") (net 4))
 (segment (start 103.975 92.1) (end 102.8 92.1) (width 0.25) (layer "F.Cu") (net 4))
 (segment (start 102.6 92.3) (end 102.6 98.6) (width 0.25) (layer "F.Cu") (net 4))
 (segment (start 109.7 91.5) (end 109.7 88) (width 0.25) (layer "F.Cu") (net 4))
 (segment (start 102.6 98.6) (end 103.1 99.1) (width 0.25) (layer "F.Cu") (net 4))
 (segment (start 105.1 80.7) (end 109.7 85.3) (width 0.25) (layer "F.Cu") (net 4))
 (segment (start 106.6 99.1) (end 107.65 100.15) (width 0.25) (layer "F.Cu") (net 4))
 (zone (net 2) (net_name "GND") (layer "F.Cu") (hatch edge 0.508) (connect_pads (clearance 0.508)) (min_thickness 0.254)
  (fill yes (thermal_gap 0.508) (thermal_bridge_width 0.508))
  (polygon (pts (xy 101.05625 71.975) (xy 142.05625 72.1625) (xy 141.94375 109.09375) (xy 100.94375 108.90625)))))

